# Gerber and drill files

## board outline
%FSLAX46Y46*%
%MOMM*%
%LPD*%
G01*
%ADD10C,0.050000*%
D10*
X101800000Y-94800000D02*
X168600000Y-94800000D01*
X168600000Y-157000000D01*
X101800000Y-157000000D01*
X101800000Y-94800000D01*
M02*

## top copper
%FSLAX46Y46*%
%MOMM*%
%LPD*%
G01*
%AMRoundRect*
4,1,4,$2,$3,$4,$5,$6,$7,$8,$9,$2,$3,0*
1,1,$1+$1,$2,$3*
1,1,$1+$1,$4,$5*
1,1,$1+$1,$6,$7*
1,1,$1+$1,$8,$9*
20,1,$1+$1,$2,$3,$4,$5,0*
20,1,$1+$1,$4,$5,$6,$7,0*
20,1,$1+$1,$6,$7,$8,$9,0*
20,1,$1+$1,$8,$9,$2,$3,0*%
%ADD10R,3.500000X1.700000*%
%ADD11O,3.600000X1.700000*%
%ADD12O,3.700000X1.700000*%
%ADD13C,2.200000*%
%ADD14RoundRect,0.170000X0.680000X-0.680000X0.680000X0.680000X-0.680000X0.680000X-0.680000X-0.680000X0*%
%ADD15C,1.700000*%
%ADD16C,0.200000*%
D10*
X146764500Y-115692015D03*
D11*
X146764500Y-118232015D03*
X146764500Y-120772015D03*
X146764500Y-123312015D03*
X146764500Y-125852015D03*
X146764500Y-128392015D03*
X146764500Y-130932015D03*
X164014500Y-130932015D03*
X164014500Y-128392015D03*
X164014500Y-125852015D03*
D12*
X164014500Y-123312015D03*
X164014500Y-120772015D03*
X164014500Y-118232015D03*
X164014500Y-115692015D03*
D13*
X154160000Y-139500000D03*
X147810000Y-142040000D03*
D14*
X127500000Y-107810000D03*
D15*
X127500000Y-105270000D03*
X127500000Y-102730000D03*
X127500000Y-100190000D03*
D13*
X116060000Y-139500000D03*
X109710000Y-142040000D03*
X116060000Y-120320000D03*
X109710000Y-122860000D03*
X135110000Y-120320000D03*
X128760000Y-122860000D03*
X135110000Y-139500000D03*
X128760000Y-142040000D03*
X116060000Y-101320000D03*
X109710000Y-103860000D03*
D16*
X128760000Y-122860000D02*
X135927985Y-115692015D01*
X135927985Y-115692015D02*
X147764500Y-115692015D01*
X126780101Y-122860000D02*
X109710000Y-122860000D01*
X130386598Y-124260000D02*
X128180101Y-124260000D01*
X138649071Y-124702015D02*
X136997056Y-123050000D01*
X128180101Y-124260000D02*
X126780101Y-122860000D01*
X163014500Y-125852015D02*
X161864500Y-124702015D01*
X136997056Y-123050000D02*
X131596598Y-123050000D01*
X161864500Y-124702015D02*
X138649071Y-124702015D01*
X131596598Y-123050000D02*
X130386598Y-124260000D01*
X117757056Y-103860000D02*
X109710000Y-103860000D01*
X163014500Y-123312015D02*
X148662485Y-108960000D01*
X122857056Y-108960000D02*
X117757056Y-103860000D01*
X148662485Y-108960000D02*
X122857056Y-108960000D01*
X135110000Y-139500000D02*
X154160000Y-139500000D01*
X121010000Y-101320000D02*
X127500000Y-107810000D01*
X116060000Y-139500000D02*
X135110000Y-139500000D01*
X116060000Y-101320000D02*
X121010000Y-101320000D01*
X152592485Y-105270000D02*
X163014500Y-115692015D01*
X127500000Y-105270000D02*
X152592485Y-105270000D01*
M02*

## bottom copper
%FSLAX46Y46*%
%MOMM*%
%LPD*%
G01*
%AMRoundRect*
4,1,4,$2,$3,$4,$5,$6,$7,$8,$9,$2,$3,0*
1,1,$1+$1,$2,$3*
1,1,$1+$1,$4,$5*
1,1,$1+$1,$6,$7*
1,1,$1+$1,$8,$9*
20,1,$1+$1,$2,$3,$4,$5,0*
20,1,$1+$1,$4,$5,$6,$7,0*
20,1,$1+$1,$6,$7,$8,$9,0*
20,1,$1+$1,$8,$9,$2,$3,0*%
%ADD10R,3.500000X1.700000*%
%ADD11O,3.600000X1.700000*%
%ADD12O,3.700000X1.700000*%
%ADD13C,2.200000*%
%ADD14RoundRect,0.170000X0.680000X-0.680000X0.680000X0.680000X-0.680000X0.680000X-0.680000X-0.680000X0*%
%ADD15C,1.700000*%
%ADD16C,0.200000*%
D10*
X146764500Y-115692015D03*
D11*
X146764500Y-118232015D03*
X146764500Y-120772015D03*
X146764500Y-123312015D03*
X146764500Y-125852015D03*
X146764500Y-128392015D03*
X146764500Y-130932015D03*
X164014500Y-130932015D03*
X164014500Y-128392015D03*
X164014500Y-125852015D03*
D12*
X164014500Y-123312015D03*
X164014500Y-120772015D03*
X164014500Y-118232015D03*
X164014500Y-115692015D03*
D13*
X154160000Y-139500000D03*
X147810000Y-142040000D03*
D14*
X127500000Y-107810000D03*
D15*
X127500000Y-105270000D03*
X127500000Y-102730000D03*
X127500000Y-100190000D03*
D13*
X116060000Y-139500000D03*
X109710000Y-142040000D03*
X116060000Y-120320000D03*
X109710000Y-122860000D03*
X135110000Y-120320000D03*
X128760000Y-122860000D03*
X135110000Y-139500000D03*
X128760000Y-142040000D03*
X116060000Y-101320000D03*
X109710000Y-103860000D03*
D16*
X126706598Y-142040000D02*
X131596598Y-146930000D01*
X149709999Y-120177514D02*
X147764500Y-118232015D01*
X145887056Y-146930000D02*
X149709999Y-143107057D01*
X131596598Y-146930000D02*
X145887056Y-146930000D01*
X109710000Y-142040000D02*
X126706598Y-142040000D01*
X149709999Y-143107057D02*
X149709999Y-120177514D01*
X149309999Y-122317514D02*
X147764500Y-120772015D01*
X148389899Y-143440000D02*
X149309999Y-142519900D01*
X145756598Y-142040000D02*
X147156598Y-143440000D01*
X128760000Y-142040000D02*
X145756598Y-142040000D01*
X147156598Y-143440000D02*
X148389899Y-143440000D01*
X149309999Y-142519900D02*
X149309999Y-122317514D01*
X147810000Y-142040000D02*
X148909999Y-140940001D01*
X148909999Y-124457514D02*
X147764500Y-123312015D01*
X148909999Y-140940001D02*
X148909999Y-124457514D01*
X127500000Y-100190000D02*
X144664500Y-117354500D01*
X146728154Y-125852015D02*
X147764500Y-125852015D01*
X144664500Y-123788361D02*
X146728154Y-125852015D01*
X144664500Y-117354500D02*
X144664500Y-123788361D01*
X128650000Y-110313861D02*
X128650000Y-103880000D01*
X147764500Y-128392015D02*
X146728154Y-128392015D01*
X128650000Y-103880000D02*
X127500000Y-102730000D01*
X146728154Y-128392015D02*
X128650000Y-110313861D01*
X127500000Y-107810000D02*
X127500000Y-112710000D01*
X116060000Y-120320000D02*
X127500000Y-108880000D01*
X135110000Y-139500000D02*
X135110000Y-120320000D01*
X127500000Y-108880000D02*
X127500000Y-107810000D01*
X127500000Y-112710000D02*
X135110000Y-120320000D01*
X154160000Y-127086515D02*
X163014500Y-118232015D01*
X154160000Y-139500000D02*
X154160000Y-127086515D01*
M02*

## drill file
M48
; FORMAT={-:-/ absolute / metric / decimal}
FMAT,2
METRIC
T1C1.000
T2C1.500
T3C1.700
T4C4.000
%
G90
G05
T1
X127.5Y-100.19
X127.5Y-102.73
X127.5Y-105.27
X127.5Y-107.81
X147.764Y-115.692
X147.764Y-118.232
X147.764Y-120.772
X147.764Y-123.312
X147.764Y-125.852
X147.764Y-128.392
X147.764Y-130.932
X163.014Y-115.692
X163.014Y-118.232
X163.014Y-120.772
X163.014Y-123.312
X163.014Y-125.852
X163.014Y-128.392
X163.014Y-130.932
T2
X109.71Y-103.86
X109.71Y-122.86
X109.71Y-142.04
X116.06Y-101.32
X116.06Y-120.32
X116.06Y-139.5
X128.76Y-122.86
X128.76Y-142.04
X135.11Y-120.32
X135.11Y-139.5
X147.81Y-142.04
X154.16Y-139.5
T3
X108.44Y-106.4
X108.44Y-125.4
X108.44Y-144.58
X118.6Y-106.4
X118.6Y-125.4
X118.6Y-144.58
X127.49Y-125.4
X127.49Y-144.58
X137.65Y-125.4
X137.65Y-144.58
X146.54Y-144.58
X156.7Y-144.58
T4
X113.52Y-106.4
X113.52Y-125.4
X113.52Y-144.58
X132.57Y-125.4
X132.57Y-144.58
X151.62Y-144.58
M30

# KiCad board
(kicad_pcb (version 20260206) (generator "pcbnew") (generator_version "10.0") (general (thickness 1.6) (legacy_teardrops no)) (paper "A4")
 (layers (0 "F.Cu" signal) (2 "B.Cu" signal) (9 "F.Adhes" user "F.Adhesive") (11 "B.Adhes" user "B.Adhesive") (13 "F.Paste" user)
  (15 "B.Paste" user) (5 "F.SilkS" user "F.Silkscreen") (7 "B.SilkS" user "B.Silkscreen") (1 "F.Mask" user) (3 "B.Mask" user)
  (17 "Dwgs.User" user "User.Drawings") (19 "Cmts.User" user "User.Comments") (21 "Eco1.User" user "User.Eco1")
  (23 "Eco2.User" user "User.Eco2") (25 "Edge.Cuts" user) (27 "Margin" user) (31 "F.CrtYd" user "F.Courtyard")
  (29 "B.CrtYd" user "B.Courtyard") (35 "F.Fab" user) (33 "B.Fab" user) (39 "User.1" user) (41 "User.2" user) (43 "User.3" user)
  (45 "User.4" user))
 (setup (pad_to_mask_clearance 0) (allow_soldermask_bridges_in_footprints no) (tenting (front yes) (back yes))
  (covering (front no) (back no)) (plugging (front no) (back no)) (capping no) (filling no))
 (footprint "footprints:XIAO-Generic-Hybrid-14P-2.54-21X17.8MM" (layer "F.Cu") (at 155.3895 123.312015)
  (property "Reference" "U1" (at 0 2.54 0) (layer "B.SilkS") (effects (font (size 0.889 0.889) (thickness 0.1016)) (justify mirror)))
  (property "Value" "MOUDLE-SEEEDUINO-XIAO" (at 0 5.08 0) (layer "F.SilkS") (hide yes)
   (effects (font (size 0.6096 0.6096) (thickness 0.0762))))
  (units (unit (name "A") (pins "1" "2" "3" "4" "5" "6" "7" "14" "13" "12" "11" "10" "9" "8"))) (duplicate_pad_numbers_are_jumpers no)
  (pad "1" thru_hole rect (at -7.625 -7.62) (size 3.5 1.7) (drill 1 (offset -1 0)) (layers "*.Cu" "*.Mask") (remove_unused_layers no)
   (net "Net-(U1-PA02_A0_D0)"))
  (pad "2" thru_hole oval (at -7.625 -5.08) (size 3.6 1.7) (drill 1 (offset -1 0)) (layers "*.Cu" "*.Mask") (remove_unused_layers no)
   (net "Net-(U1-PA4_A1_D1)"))
  (pad "3" thru_hole oval (at -7.625 -2.54) (size 3.6 1.7) (drill 1 (offset -1 0)) (layers "*.Cu" "*.Mask") (remove_unused_layers no)
   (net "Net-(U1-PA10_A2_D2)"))
  (pad "4" thru_hole oval (at -7.625 0) (size 3.6 1.7) (drill 1 (offset -1 0)) (layers "*.Cu" "*.Mask") (remove_unused_layers no)
   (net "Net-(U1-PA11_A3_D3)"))
  (pad "5" thru_hole oval (at -7.625 2.54) (size 3.6 1.7) (drill 1 (offset -1 0)) (layers "*.Cu" "*.Mask") (remove_unused_layers no)
   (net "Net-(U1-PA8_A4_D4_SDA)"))
  (pad "6" thru_hole oval (at -7.625 5.08 180) (size 3.6 1.7) (drill 1 (offset 1 0)) (layers "*.Cu" "*.Mask") (remove_unused_layers no)
   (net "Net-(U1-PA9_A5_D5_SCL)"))
  (pad "7" thru_hole oval (at -7.625 7.62) (size 3.6 1.7) (drill 1 (offset -1 0)) (layers "*.Cu" "*.Mask") (remove_unused_layers no)
   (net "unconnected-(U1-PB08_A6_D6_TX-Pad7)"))
  (pad "8" thru_hole oval (at 7.625 7.62) (size 3.6 1.7) (drill 1 (offset 1 0)) (layers "*.Cu" "*.Mask") (remove_unused_layers no)
   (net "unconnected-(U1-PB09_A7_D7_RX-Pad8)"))
  (pad "9" thru_hole oval (at 7.625 5.08) (size 3.6 1.7) (drill 1 (offset 1 0)) (layers "*.Cu" "*.Mask") (remove_unused_layers no)
   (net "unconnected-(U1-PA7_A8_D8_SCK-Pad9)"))
  (pad "10" thru_hole oval (at 7.625 2.54) (size 3.6 1.7) (drill 1 (offset 1 0)) (layers "*.Cu" "*.Mask") (remove_unused_layers no)
   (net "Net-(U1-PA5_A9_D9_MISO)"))
  (pad "11" thru_hole oval (at 7.625 0) (size 3.7 1.7) (drill 1 (offset 1 0)) (layers "*.Cu" "*.Mask") (remove_unused_layers no)
   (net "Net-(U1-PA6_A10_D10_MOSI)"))
  (pad "12" thru_hole oval (at 7.625 -2.54) (size 3.7 1.7) (drill 1 (offset 1 0)) (layers "*.Cu" "*.Mask") (remove_unused_layers no)
   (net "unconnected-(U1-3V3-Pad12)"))
  (pad "13" thru_hole oval (at 7.625 -5.08) (size 3.7 1.7) (drill 1 (offset 1 0)) (layers "*.Cu" "*.Mask") (remove_unused_layers no)
   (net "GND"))
  (pad "14" thru_hole oval (at 7.625 -7.62) (size 3.7 1.7) (drill 1 (offset 1 0)) (layers "*.Cu" "*.Mask") (remove_unused_layers no)
   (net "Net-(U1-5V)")))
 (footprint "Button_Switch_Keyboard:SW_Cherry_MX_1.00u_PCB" (layer "F.Cu") (at 154.16 139.5)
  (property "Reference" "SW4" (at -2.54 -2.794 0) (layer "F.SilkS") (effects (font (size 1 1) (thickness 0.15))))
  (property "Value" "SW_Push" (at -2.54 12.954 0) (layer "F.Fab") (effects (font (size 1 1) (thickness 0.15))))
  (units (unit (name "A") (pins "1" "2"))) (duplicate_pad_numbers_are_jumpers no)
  (pad "" np_thru_hole circle (at -7.62 5.08) (size 1.7 1.7) (drill 1.7) (layers "*.Cu" "*.Mask"))
  (pad "" np_thru_hole circle (at -2.54 5.08) (size 4 4) (drill 4) (layers "*.Cu" "*.Mask"))
  (pad "" np_thru_hole circle (at 2.54 5.08) (size 1.7 1.7) (drill 1.7) (layers "*.Cu" "*.Mask"))
  (pad "1" thru_hole circle (at 0 0) (size 2.2 2.2) (drill 1.5) (layers "*.Cu" "*.Mask") (remove_unused_layers no) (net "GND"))
  (pad "2" thru_hole circle (at -6.35 2.54) (size 2.2 2.2) (drill 1.5) (layers "*.Cu" "*.Mask") (remove_unused_layers no)
   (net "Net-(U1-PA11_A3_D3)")))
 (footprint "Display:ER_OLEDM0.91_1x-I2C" (layer "F.Cu") (at 127.5 107.81 90)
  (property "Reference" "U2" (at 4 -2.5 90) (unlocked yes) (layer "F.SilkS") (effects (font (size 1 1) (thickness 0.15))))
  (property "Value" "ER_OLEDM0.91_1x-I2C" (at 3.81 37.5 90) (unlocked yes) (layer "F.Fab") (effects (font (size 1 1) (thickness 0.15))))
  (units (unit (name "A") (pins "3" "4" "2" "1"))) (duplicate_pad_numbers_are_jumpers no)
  (pad "1" thru_hole roundrect (at 0 0 90) (size 1.7 1.7) (drill 1) (layers "*.Cu" "*.Mask") (remove_unused_layers no)
   (roundrect_rratio 0.1) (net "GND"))
  (pad "2" thru_hole circle (at 2.54 0 90) (size 1.7 1.7) (drill 1) (layers "*.Cu" "*.Mask") (remove_unused_layers no) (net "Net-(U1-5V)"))
  (pad "3" thru_hole circle (at 5.08 0 90) (size 1.7 1.7) (drill 1) (layers "*.Cu" "*.Mask") (remove_unused_layers no)
   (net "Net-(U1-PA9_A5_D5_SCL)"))
  (pad "4" thru_hole circle (at 7.62 0 90) (size 1.7 1.7) (drill 1) (layers "*.Cu" "*.Mask") (remove_unused_layers no)
   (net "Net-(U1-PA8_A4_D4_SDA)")))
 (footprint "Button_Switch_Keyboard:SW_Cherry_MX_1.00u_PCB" (layer "F.Cu") (at 116.06 139.5)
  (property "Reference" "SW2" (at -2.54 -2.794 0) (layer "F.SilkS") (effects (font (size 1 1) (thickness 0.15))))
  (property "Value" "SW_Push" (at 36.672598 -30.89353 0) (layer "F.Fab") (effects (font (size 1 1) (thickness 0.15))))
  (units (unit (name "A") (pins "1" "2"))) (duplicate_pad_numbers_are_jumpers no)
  (pad "" np_thru_hole circle (at -7.62 5.08) (size 1.7 1.7) (drill 1.7) (layers "*.Cu" "*.Mask"))
  (pad "" np_thru_hole circle (at -2.54 5.08) (size 4 4) (drill 4) (layers "*.Cu" "*.Mask"))
  (pad "" np_thru_hole circle (at 2.54 5.08) (size 1.7 1.7) (drill 1.7) (layers "*.Cu" "*.Mask"))
  (pad "1" thru_hole circle (at 0 0) (size 2.2 2.2) (drill 1.5) (layers "*.Cu" "*.Mask") (remove_unused_layers no) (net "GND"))
  (pad "2" thru_hole circle (at -6.35 2.54) (size 2.2 2.2) (drill 1.5) (layers "*.Cu" "*.Mask") (remove_unused_layers no)
   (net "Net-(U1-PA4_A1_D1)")))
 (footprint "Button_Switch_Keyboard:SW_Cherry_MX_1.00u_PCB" (layer "F.Cu") (at 116.06 120.32)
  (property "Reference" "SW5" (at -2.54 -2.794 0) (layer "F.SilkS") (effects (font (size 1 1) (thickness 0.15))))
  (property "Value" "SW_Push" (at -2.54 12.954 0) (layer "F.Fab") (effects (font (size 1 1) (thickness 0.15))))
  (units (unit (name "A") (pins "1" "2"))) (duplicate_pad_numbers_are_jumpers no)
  (pad "" np_thru_hole circle (at -7.62 5.08) (size 1.7 1.7) (drill 1.7) (layers "*.Cu" "*.Mask"))
  (pad "" np_thru_hole circle (at -2.54 5.08) (size 4 4) (drill 4) (layers "*.Cu" "*.Mask"))
  (pad "" np_thru_hole circle (at 2.54 5.08) (size 1.7 1.7) (drill 1.7) (layers "*.Cu" "*.Mask"))
  (pad "1" thru_hole circle (at 0 0) (size 2.2 2.2) (drill 1.5) (layers "*.Cu" "*.Mask") (remove_unused_layers no) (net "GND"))
  (pad "2" thru_hole circle (at -6.35 2.54) (size 2.2 2.2) (drill 1.5) (layers "*.Cu" "*.Mask") (remove_unused_layers no)
   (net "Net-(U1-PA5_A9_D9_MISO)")))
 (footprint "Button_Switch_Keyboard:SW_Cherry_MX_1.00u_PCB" (layer "F.Cu") (at 135.11 120.32)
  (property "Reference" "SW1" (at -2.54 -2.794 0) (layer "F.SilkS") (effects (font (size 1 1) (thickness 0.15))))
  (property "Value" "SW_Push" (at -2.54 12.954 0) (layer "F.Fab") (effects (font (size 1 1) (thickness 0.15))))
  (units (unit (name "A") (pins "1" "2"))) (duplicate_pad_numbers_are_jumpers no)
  (pad "" np_thru_hole circle (at -7.62 5.08) (size 1.7 1.7) (drill 1.7) (layers "*.Cu" "*.Mask"))
  (pad "" np_thru_hole circle (at -2.54 5.08) (size 4 4) (drill 4) (layers "*.Cu" "*.Mask"))
  (pad "" np_thru_hole circle (at 2.54 5.08) (size 1.7 1.7) (drill 1.7) (layers "*.Cu" "*.Mask"))
  (pad "1" thru_hole circle (at 0 0) (size 2.2 2.2) (drill 1.5) (layers "*.Cu" "*.Mask") (remove_unused_layers no) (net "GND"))
  (pad "2" thru_hole circle (at -6.35 2.54) (size 2.2 2.2) (drill 1.5) (layers "*.Cu" "*.Mask") (remove_unused_layers no)
   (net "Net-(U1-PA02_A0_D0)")))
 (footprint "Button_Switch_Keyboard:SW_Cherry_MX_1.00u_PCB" (layer "F.Cu") (at 135.11 139.5)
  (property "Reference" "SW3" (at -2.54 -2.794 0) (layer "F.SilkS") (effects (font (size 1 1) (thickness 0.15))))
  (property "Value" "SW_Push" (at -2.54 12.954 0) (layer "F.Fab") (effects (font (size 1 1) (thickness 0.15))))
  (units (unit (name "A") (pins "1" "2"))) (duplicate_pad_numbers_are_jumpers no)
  (pad "" np_thru_hole circle (at -7.62 5.08) (size 1.7 1.7) (drill 1.7) (layers "*.Cu" "*.Mask"))
  (pad "" np_thru_hole circle (at -2.54 5.08) (size 4 4) (drill 4) (layers "*.Cu" "*.Mask"))
  (pad "" np_thru_hole circle (at 2.54 5.08) (size 1.7 1.7) (drill 1.7) (layers "*.Cu" "*.Mask"))
  (pad "1" thru_hole circle (at 0 0) (size 2.2 2.2) (drill 1.5) (layers "*.Cu" "*.Mask") (remove_unused_layers no) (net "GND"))
  (pad "2" thru_hole circle (at -6.35 2.54) (size 2.2 2.2) (drill 1.5) (layers "*.Cu" "*.Mask") (remove_unused_layers no)
   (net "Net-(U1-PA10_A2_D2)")))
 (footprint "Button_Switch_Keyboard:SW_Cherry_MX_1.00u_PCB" (layer "F.Cu") (at 116.06 101.32)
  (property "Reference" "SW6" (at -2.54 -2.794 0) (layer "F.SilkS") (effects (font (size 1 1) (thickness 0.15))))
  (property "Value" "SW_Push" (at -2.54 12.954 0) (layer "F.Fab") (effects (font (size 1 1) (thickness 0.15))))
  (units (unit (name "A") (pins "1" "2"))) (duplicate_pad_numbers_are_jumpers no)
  (pad "" np_thru_hole circle (at -7.62 5.08) (size 1.7 1.7) (drill 1.7) (layers "*.Cu" "*.Mask"))
  (pad "" np_thru_hole circle (at -2.54 5.08) (size 4 4) (drill 4) (layers "*.Cu" "*.Mask"))
  (pad "" np_thru_hole circle (at 2.54 5.08) (size 1.7 1.7) (drill 1.7) (layers "*.Cu" "*.Mask"))
  (pad "1" thru_hole circle (at 0 0) (size 2.2 2.2) (drill 1.5) (layers "*.Cu" "*.Mask") (remove_unused_layers no) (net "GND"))
  (pad "2" thru_hole circle (at -6.35 2.54) (size 2.2 2.2) (drill 1.5) (layers "*.Cu" "*.Mask") (remove_unused_layers no)
   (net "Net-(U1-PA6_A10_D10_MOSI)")))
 (gr_rect (start 101.8 94.8) (end 168.6 157) (stroke (width 0.05) (type default)) (fill no) (layer "Edge.Cuts"))
 (segment (start 128.76 122.86) (end 135.927985 115.692015) (width 0.2) (layer "F.Cu") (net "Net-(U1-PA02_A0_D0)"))
 (segment (start 135.927985 115.692015) (end 147.7645 115.692015) (width 0.2) (layer "F.Cu") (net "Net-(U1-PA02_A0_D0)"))
 (segment (start 126.706598 142.04) (end 131.596598 146.93) (width 0.2) (layer "B.Cu") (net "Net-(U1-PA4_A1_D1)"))
 (segment (start 149.709999 120.177514) (end 147.7645 118.232015) (width 0.2) (layer "B.Cu") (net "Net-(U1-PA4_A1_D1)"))
 (segment (start 145.887056 146.93) (end 149.709999 143.107057) (width 0.2) (layer "B.Cu") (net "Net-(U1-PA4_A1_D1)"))
 (segment (start 131.596598 146.93) (end 145.887056 146.93) (width 0.2) (layer "B.Cu") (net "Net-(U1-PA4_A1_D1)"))
 (segment (start 109.71 142.04) (end 126.706598 142.04) (width 0.2) (layer "B.Cu") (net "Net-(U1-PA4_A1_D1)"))
 (segment (start 149.709999 143.107057) (end 149.709999 120.177514) (width 0.2) (layer "B.Cu") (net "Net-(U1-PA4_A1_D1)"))
 (segment (start 149.309999 122.317514) (end 147.7645 120.772015) (width 0.2) (layer "B.Cu") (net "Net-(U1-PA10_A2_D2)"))
 (segment (start 148.389899 143.44) (end 149.309999 142.5199) (width 0.2) (layer "B.Cu") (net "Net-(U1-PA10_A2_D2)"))
 (segment (start 145.756598 142.04) (end 147.156598 143.44) (width 0.2) (layer "B.Cu") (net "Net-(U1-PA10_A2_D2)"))
 (segment (start 128.76 142.04) (end 145.756598 142.04) (width 0.2) (layer "B.Cu") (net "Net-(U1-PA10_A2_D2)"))
 (segment (start 147.156598 143.44) (end 148.389899 143.44) (width 0.2) (layer "B.Cu") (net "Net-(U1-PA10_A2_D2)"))
 (segment (start 149.309999 142.5199) (end 149.309999 122.317514) (width 0.2) (layer "B.Cu") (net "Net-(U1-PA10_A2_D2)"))
 (segment (start 147.81 142.04) (end 148.909999 140.940001) (width 0.2) (layer "B.Cu") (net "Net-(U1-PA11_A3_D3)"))
 (segment (start 148.909999 124.457514) (end 147.7645 123.312015) (width 0.2) (layer "B.Cu") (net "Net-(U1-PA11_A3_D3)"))
 (segment (start 148.909999 140.940001) (end 148.909999 124.457514) (width 0.2) (layer "B.Cu") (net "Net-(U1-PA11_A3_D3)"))
 (segment (start 127.5 100.19) (end 144.6645 117.3545) (width 0.2) (layer "B.Cu") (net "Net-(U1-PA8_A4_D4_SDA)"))
 (segment (start 146.728154 125.852015) (end 147.7645 125.852015) (width 0.2) (layer "B.Cu") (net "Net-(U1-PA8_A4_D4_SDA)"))
 (segment (start 144.6645 123.788361) (end 146.728154 125.852015) (width 0.2) (layer "B.Cu") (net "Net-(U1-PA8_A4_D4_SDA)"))
 (segment (start 144.6645 117.3545) (end 144.6645 123.788361) (width 0.2) (layer "B.Cu") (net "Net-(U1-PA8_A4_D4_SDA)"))
 (segment (start 128.65 110.313861) (end 128.65 103.88) (width 0.2) (layer "B.Cu") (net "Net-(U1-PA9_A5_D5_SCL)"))
 (segment (start 147.7645 128.392015) (end 146.728154 128.392015) (width 0.2) (layer "B.Cu") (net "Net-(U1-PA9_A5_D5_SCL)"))
 (segment (start 128.65 103.88) (end 127.5 102.73) (width 0.2) (layer "B.Cu") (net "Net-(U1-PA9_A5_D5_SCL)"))
 (segment (start 146.728154 128.392015) (end 128.65 110.313861) (width 0.2) (layer "B.Cu") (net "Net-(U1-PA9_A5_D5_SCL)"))
 (segment (start 126.780101 122.86) (end 109.71 122.86) (width 0.2) (layer "F.Cu") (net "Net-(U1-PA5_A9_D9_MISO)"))
 (segment (start 130.386598 124.26) (end 128.180101 124.26) (width 0.2) (layer "F.Cu") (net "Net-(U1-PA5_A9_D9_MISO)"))
 (segment (start 138.649071 124.702015) (end 136.997056 123.05) (width 0.2) (layer "F.Cu") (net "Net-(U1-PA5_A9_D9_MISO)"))
 (segment (start 128.180101 124.26) (end 126.780101 122.86) (width 0.2) (layer "F.Cu") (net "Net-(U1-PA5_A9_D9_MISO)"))
 (segment (start 163.0145 125.852015) (end 161.8645 124.702015) (width 0.2) (layer "F.Cu") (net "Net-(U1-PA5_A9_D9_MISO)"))
 (segment (start 136.997056 123.05) (end 131.596598 123.05) (width 0.2) (layer "F.Cu") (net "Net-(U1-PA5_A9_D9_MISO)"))
 (segment (start 161.8645 124.702015) (end 138.649071 124.702015) (width 0.2) (layer "F.Cu") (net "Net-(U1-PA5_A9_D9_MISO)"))
 (segment (start 131.596598 123.05) (end 130.386598 124.26) (width 0.2) (layer "F.Cu") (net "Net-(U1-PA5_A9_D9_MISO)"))
 (segment (start 117.757056 103.86) (end 109.71 103.86) (width 0.2) (layer "F.Cu") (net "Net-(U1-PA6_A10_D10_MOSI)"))
 (segment (start 163.0145 123.312015) (end 148.662485 108.96) (width 0.2) (layer "F.Cu") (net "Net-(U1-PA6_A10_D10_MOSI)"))
 (segment (start 122.857056 108.96) (end 117.757056 103.86) (width 0.2) (layer "F.Cu") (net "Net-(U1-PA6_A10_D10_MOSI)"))
 (segment (start 148.662485 108.96) (end 122.857056 108.96) (width 0.2) (layer "F.Cu") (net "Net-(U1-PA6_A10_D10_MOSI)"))
 (segment (start 135.11 139.5) (end 154.16 139.5) (width 0.2) (layer "F.Cu") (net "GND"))
 (segment (start 121.01 101.32) (end 127.5 107.81) (width 0.2) (layer "F.Cu") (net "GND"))
 (segment (start 116.06 139.5) (end 135.11 139.5) (width 0.2) (layer "F.Cu") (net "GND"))
 (segment (start 116.06 101.32) (end 121.01 101.32) (width 0.2) (layer "F.Cu") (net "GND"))
 (segment (start 127.5 107.81) (end 127.5 112.71) (width 0.2) (layer "B.Cu") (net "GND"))
 (segment (start 116.06 120.32) (end 127.5 108.88) (width 0.2) (layer "B.Cu") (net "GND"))
 (segment (start 135.11 139.5) (end 135.11 120.32) (width 0.2) (layer "B.Cu") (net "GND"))
 (segment (start 127.5 108.88) (end 127.5 107.81) (width 0.2) (layer "B.Cu") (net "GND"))
 (segment (start 127.5 112.71) (end 135.11 120.32) (width 0.2) (layer "B.Cu") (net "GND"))
 (segment (start 154.16 127.086515) (end 163.0145 118.232015) (width 0.2) (layer "B.Cu") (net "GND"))
 (segment (start 154.16 139.5) (end 154.16 127.086515) (width 0.2) (layer "B.Cu") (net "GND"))
 (segment (start 152.592485 105.27) (end 163.0145 115.692015) (width 0.2) (layer "F.Cu") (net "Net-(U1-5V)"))
 (segment (start 127.5 105.27) (end 152.592485 105.27) (width 0.2) (layer "F.Cu") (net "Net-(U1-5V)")))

